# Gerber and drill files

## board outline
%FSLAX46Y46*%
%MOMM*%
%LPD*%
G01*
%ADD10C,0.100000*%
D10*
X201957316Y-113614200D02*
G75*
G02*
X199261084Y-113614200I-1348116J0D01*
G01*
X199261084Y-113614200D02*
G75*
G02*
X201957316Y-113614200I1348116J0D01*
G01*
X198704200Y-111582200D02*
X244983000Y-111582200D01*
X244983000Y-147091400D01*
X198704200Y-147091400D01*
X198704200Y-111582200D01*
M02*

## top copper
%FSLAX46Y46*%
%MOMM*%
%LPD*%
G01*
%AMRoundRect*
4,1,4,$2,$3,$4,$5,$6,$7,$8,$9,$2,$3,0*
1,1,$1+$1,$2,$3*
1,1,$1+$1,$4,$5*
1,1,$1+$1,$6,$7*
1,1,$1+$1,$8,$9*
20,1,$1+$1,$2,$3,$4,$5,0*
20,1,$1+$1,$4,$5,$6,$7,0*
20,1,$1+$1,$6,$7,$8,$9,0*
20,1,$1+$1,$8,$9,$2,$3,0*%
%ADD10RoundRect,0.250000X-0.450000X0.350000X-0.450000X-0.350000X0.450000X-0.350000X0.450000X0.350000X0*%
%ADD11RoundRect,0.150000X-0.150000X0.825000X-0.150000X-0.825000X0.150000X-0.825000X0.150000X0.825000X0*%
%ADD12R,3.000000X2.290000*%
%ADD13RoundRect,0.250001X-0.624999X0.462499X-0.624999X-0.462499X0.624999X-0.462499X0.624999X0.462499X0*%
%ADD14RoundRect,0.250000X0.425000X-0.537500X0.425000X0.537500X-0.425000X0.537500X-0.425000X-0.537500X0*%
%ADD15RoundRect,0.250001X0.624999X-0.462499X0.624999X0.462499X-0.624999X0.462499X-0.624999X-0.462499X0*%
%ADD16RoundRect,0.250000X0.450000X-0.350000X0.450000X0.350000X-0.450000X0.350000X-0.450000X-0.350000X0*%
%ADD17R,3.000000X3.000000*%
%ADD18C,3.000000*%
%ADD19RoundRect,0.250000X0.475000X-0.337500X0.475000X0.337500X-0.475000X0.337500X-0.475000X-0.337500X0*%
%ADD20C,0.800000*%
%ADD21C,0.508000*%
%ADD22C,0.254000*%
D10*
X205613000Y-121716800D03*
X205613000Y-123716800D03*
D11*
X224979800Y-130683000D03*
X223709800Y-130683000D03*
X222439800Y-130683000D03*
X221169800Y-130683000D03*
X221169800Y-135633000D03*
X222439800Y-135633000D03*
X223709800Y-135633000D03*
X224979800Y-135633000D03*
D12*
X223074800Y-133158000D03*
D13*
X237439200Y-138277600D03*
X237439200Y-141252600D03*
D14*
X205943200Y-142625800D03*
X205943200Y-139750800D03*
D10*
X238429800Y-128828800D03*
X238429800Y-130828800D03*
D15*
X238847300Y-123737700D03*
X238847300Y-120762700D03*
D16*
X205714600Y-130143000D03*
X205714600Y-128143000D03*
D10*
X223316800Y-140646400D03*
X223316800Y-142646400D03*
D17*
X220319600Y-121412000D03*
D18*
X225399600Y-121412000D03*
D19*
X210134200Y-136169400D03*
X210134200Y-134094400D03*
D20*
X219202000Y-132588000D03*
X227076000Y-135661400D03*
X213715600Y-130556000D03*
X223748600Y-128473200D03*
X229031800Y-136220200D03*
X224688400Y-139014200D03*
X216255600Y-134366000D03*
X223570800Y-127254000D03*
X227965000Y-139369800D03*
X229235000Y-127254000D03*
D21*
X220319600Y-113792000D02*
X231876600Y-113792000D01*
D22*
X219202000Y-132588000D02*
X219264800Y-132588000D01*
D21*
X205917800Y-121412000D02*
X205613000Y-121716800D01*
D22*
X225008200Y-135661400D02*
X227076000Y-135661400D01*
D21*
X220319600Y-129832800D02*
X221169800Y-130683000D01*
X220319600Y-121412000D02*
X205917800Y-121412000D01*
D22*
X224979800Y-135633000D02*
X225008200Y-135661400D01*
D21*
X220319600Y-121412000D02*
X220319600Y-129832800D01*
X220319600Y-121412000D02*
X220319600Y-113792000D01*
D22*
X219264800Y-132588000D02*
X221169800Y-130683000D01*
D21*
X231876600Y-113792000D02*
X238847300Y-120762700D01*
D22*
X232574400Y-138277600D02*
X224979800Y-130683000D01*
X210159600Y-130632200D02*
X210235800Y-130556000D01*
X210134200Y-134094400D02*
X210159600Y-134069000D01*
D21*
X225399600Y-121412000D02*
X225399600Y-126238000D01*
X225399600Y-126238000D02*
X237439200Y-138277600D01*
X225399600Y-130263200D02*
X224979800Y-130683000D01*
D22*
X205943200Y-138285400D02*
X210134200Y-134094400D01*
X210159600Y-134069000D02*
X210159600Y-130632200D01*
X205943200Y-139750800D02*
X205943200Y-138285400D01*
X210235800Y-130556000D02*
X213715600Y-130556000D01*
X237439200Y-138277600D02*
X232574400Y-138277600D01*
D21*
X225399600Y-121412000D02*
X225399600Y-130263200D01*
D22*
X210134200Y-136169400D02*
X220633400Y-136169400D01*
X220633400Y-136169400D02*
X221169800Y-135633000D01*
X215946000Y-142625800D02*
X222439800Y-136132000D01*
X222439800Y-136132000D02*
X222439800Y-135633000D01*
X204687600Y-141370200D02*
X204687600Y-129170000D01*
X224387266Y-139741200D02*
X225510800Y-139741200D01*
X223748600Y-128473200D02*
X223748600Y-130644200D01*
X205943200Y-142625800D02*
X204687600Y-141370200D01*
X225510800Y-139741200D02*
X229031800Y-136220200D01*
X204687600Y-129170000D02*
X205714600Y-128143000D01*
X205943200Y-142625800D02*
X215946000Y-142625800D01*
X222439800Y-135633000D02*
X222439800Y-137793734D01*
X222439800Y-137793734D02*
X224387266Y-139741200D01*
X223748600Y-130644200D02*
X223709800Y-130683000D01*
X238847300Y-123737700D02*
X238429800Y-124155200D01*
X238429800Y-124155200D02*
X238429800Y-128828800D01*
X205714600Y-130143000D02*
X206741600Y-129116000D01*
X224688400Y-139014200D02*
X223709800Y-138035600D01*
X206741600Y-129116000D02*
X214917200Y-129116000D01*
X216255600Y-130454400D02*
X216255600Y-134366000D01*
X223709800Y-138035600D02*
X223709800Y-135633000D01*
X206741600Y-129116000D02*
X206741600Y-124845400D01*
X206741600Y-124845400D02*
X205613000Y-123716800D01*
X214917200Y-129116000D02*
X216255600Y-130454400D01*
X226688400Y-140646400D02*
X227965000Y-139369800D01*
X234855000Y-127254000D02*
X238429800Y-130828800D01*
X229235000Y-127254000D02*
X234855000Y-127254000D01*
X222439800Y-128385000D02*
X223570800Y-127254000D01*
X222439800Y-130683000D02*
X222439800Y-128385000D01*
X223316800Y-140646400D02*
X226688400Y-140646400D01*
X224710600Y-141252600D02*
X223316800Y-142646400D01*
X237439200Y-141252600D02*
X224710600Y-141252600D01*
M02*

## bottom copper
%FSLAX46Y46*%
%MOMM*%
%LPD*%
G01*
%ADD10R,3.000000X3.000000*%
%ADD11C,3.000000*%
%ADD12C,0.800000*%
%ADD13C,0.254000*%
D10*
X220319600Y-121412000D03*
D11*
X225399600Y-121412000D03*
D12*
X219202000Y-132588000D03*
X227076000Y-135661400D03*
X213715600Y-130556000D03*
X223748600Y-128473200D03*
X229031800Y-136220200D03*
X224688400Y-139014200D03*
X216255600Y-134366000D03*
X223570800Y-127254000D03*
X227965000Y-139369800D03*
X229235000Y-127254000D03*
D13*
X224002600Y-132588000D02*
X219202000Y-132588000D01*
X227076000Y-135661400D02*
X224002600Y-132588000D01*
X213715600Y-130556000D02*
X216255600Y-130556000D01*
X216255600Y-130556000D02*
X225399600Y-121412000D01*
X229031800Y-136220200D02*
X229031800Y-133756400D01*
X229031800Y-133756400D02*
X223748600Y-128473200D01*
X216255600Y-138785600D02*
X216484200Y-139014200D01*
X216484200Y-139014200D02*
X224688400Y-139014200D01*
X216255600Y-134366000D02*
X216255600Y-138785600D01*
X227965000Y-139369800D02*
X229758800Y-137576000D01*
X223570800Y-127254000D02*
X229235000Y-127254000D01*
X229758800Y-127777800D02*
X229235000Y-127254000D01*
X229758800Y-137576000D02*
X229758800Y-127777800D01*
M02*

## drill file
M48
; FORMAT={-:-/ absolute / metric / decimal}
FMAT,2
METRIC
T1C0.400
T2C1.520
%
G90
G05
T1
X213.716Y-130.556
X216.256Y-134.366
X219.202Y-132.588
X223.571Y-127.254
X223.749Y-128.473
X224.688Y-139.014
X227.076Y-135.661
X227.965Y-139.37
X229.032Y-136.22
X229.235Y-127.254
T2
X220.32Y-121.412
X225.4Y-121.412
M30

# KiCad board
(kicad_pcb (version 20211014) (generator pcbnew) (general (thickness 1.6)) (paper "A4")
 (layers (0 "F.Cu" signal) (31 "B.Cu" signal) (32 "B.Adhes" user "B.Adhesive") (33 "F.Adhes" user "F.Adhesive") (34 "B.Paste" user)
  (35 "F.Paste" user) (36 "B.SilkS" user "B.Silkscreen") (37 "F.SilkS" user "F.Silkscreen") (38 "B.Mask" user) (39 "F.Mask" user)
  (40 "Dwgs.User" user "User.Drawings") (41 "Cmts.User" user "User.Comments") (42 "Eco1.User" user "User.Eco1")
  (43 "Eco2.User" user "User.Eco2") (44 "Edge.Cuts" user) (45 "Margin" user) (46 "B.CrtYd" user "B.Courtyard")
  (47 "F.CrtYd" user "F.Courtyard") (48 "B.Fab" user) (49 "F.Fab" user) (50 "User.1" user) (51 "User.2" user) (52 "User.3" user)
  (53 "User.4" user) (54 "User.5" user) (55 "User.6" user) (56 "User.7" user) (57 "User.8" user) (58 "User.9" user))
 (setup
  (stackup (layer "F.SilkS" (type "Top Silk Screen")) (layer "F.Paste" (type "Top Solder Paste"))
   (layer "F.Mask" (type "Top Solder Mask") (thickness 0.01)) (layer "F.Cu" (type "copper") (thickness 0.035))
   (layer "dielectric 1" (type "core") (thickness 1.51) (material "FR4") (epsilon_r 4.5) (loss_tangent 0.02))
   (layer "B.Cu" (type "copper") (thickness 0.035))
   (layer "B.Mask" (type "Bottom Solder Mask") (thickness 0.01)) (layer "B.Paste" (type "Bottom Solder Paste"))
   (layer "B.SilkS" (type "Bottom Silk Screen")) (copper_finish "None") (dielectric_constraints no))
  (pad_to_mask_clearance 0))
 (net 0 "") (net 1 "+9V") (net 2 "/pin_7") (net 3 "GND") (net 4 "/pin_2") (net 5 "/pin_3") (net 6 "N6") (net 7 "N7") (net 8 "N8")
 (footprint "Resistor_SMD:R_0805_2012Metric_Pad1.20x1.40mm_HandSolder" (layer "F.Cu") (at 205.613 122.7168 -90)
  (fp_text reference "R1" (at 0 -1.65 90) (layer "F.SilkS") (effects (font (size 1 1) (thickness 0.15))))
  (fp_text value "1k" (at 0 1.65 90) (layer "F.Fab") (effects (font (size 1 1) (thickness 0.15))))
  (pad "1" smd roundrect (at -1 0 270) (size 1.2 1.4) (layers "F.Cu" "F.Paste" "F.Mask") (roundrect_rratio 0.2083333333) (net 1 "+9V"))
  (pad "2" smd roundrect (at 1 0 270) (size 1.2 1.4) (layers "F.Cu" "F.Paste" "F.Mask") (roundrect_rratio 0.2083333333) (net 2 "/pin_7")))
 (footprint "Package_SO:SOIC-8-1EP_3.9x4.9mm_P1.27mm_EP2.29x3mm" (layer "F.Cu") (at 223.0748 133.158 -90)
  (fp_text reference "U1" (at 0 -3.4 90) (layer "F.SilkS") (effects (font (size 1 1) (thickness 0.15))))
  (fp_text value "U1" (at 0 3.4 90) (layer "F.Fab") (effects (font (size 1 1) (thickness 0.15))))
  (pad "" smd roundrect (at 0.57 -0.75 270) (size 0.92 1.21) (layers "F.Paste") (roundrect_rratio 0.25))
  (pad "" smd roundrect (at -0.57 0.75 270) (size 0.92 1.21) (layers "F.Paste") (roundrect_rratio 0.25))
  (pad "" smd roundrect (at 0.57 0.75 270) (size 0.92 1.21) (layers "F.Paste") (roundrect_rratio 0.25))
  (pad "" smd roundrect (at -0.57 -0.75 270) (size 0.92 1.21) (layers "F.Paste") (roundrect_rratio 0.25))
  (pad "1" smd roundrect (at -2.475 -1.905 270) (size 1.95 0.6) (layers "F.Cu" "F.Paste" "F.Mask") (roundrect_rratio 0.25) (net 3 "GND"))
  (pad "2" smd roundrect (at -2.475 -0.635 270) (size 1.95 0.6) (layers "F.Cu" "F.Paste" "F.Mask") (roundrect_rratio 0.25) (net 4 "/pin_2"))
  (pad "3" smd roundrect (at -2.475 0.635 270) (size 1.95 0.6) (layers "F.Cu" "F.Paste" "F.Mask") (roundrect_rratio 0.25) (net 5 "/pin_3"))
  (pad "4" smd roundrect (at -2.475 1.905 270) (size 1.95 0.6) (layers "F.Cu" "F.Paste" "F.Mask") (roundrect_rratio 0.25) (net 1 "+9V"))
  (pad "5" smd roundrect (at 2.475 1.905 270) (size 1.95 0.6) (layers "F.Cu" "F.Paste" "F.Mask") (roundrect_rratio 0.25) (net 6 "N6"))
  (pad "6" smd roundrect (at 2.475 0.635 270) (size 1.95 0.6) (layers "F.Cu" "F.Paste" "F.Mask") (roundrect_rratio 0.25) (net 4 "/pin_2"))
  (pad "7" smd roundrect (at 2.475 -0.635 270) (size 1.95 0.6) (layers "F.Cu" "F.Paste" "F.Mask") (roundrect_rratio 0.25) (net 2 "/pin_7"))
  (pad "8" smd roundrect (at 2.475 -1.905 270) (size 1.95 0.6) (layers "F.Cu" "F.Paste" "F.Mask") (roundrect_rratio 0.25) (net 1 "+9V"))
  (pad "9" smd rect (at 0 0 270) (size 2.29 3) (layers "F.Cu" "F.Mask")))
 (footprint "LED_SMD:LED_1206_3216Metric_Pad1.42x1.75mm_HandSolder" (layer "F.Cu") (at 237.4392 139.7651 -90)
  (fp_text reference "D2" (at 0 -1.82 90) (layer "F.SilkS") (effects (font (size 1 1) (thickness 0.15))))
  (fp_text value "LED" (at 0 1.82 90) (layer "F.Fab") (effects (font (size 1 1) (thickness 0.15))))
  (pad "1" smd roundrect (at -1.4875 0 270) (size 1.425 1.75) (layers "F.Cu" "F.Paste" "F.Mask") (roundrect_rratio 0.1754392982)
   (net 3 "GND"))
  (pad "2" smd roundrect (at 1.4875 0 270) (size 1.425 1.75) (layers "F.Cu" "F.Paste" "F.Mask") (roundrect_rratio 0.1754392982) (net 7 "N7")))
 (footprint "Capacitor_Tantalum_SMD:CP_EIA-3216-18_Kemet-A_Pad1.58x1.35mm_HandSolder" (layer "F.Cu") (at 205.9432 141.1883 90)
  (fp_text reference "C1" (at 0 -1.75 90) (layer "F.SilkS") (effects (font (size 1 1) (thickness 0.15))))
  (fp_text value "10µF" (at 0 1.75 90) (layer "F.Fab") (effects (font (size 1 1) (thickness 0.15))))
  (pad "1" smd roundrect (at -1.4375 0 90) (size 1.575 1.35) (layers "F.Cu" "F.Paste" "F.Mask") (roundrect_rratio 0.1851851852)
   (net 4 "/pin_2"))
  (pad "2" smd roundrect (at 1.4375 0 90) (size 1.575 1.35) (layers "F.Cu" "F.Paste" "F.Mask") (roundrect_rratio 0.1851851852) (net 3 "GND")))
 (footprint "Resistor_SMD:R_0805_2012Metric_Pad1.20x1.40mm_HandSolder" (layer "F.Cu") (at 238.4298 129.8288 -90)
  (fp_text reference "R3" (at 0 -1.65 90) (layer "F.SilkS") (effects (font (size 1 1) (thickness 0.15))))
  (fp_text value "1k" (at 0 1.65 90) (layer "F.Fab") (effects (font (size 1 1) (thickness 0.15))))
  (pad "1" smd roundrect (at -1 0 270) (size 1.2 1.4) (layers "F.Cu" "F.Paste" "F.Mask") (roundrect_rratio 0.2083333333) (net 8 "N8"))
  (pad "2" smd roundrect (at 1 0 270) (size 1.2 1.4) (layers "F.Cu" "F.Paste" "F.Mask") (roundrect_rratio 0.2083333333) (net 5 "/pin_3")))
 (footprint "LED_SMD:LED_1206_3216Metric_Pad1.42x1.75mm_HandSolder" (layer "F.Cu") (at 238.8473 122.2502 90)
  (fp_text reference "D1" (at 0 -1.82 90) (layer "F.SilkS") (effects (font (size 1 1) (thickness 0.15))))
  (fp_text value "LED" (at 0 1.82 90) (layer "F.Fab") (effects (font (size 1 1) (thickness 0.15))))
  (pad "1" smd roundrect (at -1.4875 0 90) (size 1.425 1.75) (layers "F.Cu" "F.Paste" "F.Mask") (roundrect_rratio 0.1754392982) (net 8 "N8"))
  (pad "2" smd roundrect (at 1.4875 0 90) (size 1.425 1.75) (layers "F.Cu" "F.Paste" "F.Mask") (roundrect_rratio 0.1754392982) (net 1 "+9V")))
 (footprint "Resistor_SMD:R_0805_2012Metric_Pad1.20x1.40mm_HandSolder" (layer "F.Cu") (at 205.7146 129.143 90)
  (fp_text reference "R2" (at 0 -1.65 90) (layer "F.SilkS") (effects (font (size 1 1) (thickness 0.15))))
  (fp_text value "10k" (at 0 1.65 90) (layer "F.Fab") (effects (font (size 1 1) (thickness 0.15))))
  (pad "1" smd roundrect (at -1 0 90) (size 1.2 1.4) (layers "F.Cu" "F.Paste" "F.Mask") (roundrect_rratio 0.2083333333) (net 2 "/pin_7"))
  (pad "2" smd roundrect (at 1 0 90) (size 1.2 1.4) (layers "F.Cu" "F.Paste" "F.Mask") (roundrect_rratio 0.2083333333) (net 4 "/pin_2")))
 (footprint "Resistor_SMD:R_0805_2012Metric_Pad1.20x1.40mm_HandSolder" (layer "F.Cu") (at 223.3168 141.6464 -90)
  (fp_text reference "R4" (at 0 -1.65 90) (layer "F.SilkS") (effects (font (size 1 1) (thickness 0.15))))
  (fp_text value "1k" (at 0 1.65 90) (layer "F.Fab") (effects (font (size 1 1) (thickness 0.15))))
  (pad "1" smd roundrect (at -1 0 270) (size 1.2 1.4) (layers "F.Cu" "F.Paste" "F.Mask") (roundrect_rratio 0.2083333333) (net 5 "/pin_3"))
  (pad "2" smd roundrect (at 1 0 270) (size 1.2 1.4) (layers "F.Cu" "F.Paste" "F.Mask") (roundrect_rratio 0.2083333333) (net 7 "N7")))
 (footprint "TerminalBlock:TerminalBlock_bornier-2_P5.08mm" (layer "F.Cu") (at 220.3196 121.412)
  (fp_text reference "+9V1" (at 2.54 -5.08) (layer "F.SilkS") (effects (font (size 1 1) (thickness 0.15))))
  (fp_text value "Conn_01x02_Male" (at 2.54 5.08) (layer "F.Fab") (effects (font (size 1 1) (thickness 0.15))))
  (pad "1" thru_hole rect (at 0 0) (size 3 3) (drill 1.52) (layers *.Cu *.Mask) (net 1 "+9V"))
  (pad "2" thru_hole circle (at 5.08 0) (size 3 3) (drill 1.52) (layers *.Cu *.Mask) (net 3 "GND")))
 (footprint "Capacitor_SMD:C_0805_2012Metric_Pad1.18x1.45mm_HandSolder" (layer "F.Cu") (at 210.1342 135.1319 90)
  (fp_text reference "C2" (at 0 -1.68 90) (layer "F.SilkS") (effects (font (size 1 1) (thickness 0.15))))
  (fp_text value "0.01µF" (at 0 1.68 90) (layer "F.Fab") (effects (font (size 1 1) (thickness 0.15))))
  (pad "1" smd roundrect (at -1.0375 0 90) (size 1.175 1.45) (layers "F.Cu" "F.Paste" "F.Mask") (roundrect_rratio 0.2127659574) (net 6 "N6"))
  (pad "2" smd roundrect (at 1.0375 0 90) (size 1.175 1.45) (layers "F.Cu" "F.Paste" "F.Mask") (roundrect_rratio 0.2127659574) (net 3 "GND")))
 (gr_circle (center 200.6092 113.6142) (end 201.957316 113.6142) (layer "Edge.Cuts") (width 0.1) (fill none))
 (gr_rect (start 198.7042 111.5822) (end 244.983 147.0914) (layer "Edge.Cuts") (width 0.1) (fill none))
 (segment (start 220.3196 113.792) (end 231.8766 113.792) (width 0.508) (layer "F.Cu") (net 1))
 (segment (start 219.202 132.588) (end 219.2648 132.588) (width 0.254) (layer "F.Cu") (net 1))
 (segment (start 205.9178 121.412) (end 205.613 121.7168) (width 0.508) (layer "F.Cu") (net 1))
 (segment (start 225.0082 135.6614) (end 227.076 135.6614) (width 0.254) (layer "F.Cu") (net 1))
 (segment (start 220.3196 129.8328) (end 221.1698 130.683) (width 0.508) (layer "F.Cu") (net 1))
 (segment (start 220.3196 121.412) (end 205.9178 121.412) (width 0.508) (layer "F.Cu") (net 1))
 (segment (start 224.9798 135.633) (end 225.0082 135.6614) (width 0.254) (layer "F.Cu") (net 1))
 (segment (start 220.3196 121.412) (end 220.3196 129.8328) (width 0.508) (layer "F.Cu") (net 1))
 (segment (start 220.3196 121.412) (end 220.3196 113.792) (width 0.508) (layer "F.Cu") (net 1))
 (segment (start 219.2648 132.588) (end 221.1698 130.683) (width 0.254) (layer "F.Cu") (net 1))
 (segment (start 231.8766 113.792) (end 238.8473 120.7627) (width 0.508) (layer "F.Cu") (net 1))
 (via (at 219.202 132.588) (size 0.8) (drill 0.4) (layers "F.Cu" "B.Cu") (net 1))
 (via (at 227.076 135.6614) (size 0.8) (drill 0.4) (layers "F.Cu" "B.Cu") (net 1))
 (segment (start 224.0026 132.588) (end 219.202 132.588) (width 0.254) (layer "B.Cu") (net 1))
 (segment (start 227.076 135.6614) (end 224.0026 132.588) (width 0.254) (layer "B.Cu") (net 1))
 (segment (start 232.5744 138.2776) (end 224.9798 130.683) (width 0.254) (layer "F.Cu") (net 3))
 (segment (start 210.1596 130.6322) (end 210.2358 130.556) (width 0.254) (layer "F.Cu") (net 3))
 (segment (start 210.1342 134.0944) (end 210.1596 134.069) (width 0.254) (layer "F.Cu") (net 3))
 (segment (start 225.3996 121.412) (end 225.3996 126.238) (width 0.508) (layer "F.Cu") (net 3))
 (segment (start 225.3996 126.238) (end 237.4392 138.2776) (width 0.508) (layer "F.Cu") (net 3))
 (segment (start 225.3996 130.2632) (end 224.9798 130.683) (width 0.508) (layer "F.Cu") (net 3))
 (segment (start 205.9432 138.2854) (end 210.1342 134.0944) (width 0.254) (layer "F.Cu") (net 3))
 (segment (start 210.1596 134.069) (end 210.1596 130.6322) (width 0.254) (layer "F.Cu") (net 3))
 (segment (start 205.9432 139.7508) (end 205.9432 138.2854) (width 0.254) (layer "F.Cu") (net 3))
 (segment (start 210.2358 130.556) (end 213.7156 130.556) (width 0.254) (layer "F.Cu") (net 3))
 (segment (start 237.4392 138.2776) (end 232.5744 138.2776) (width 0.254) (layer "F.Cu") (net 3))
 (segment (start 225.3996 121.412) (end 225.3996 130.2632) (width 0.508) (layer "F.Cu") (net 3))
 (via (at 213.7156 130.556) (size 0.8) (drill 0.4) (layers "F.Cu" "B.Cu") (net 3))
 (segment (start 213.7156 130.556) (end 216.2556 130.556) (width 0.254) (layer "B.Cu") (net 3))
 (segment (start 216.2556 130.556) (end 225.3996 121.412) (width 0.254) (layer "B.Cu") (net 3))
 (segment (start 210.1342 136.1694) (end 220.6334 136.1694) (width 0.254) (layer "F.Cu") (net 6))
 (segment (start 220.6334 136.1694) (end 221.1698 135.633) (width 0.254) (layer "F.Cu") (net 6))
 (segment (start 215.946 142.6258) (end 222.4398 136.132) (width 0.254) (layer "F.Cu") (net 4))
 (segment (start 222.4398 136.132) (end 222.4398 135.633) (width 0.254) (layer "F.Cu") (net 4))
 (segment (start 204.6876 141.3702) (end 204.6876 129.17) (width 0.254) (layer "F.Cu") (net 4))
 (segment (start 224.387266 139.7412) (end 225.5108 139.7412) (width 0.254) (layer "F.Cu") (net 4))
 (segment (start 223.7486 128.4732) (end 223.7486 130.6442) (width 0.254) (layer "F.Cu") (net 4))
 (segment (start 205.9432 142.6258) (end 204.6876 141.3702) (width 0.254) (layer "F.Cu") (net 4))
 (segment (start 225.5108 139.7412) (end 229.0318 136.2202) (width 0.254) (layer "F.Cu") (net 4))
 (segment (start 204.6876 129.17) (end 205.7146 128.143) (width 0.254) (layer "F.Cu") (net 4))
 (segment (start 205.9432 142.6258) (end 215.946 142.6258) (width 0.254) (layer "F.Cu") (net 4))
 (segment (start 222.4398 135.633) (end 222.4398 137.793734) (width 0.254) (layer "F.Cu") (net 4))
 (segment (start 222.4398 137.793734) (end 224.387266 139.7412) (width 0.254) (layer "F.Cu") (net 4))
 (segment (start 223.7486 130.6442) (end 223.7098 130.683) (width 0.254) (layer "F.Cu") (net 4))
 (via (at 223.7486 128.4732) (size 0.8) (drill 0.4) (layers "F.Cu" "B.Cu") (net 4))
 (via (at 229.0318 136.2202) (size 0.8) (drill 0.4) (layers "F.Cu" "B.Cu") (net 4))
 (segment (start 229.0318 136.2202) (end 229.0318 133.7564) (width 0.254) (layer "B.Cu") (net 4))
 (segment (start 229.0318 133.7564) (end 223.7486 128.4732) (width 0.254) (layer "B.Cu") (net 4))
 (segment (start 238.8473 123.7377) (end 238.4298 124.1552) (width 0.254) (layer "F.Cu") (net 8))
 (segment (start 238.4298 124.1552) (end 238.4298 128.8288) (width 0.254) (layer "F.Cu") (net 8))
 (segment (start 205.7146 130.143) (end 206.7416 129.116) (width 0.254) (layer "F.Cu") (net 2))
 (segment (start 224.6884 139.0142) (end 223.7098 138.0356) (width 0.254) (layer "F.Cu") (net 2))
 (segment (start 206.7416 129.116) (end 214.9172 129.116) (width 0.254) (layer "F.Cu") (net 2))
 (segment (start 216.2556 130.4544) (end 216.2556 134.366) (width 0.254) (layer "F.Cu") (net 2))
 (segment (start 223.7098 138.0356) (end 223.7098 135.633) (width 0.254) (layer "F.Cu") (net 2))
 (segment (start 206.7416 129.116) (end 206.7416 124.8454) (width 0.254) (layer "F.Cu") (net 2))
 (segment (start 206.7416 124.8454) (end 205.613 123.7168) (width 0.254) (layer "F.Cu") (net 2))
 (segment (start 214.9172 129.116) (end 216.2556 130.4544) (width 0.254) (layer "F.Cu") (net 2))
 (via (at 224.6884 139.0142) (size 0.8) (drill 0.4) (layers "F.Cu" "B.Cu") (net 2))
 (via (at 216.2556 134.366) (size 0.8) (drill 0.4) (layers "F.Cu" "B.Cu") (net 2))
 (segment (start 216.2556 138.7856) (end 216.4842 139.0142) (width 0.254) (layer "B.Cu") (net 2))
 (segment (start 216.4842 139.0142) (end 224.6884 139.0142) (width 0.254) (layer "B.Cu") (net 2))
 (segment (start 216.2556 134.366) (end 216.2556 138.7856) (width 0.254) (layer "B.Cu") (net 2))
 (segment (start 226.6884 140.6464) (end 227.965 139.3698) (width 0.254) (layer "F.Cu") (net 5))
 (segment (start 234.855 127.254) (end 238.4298 130.8288) (width 0.254) (layer "F.Cu") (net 5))
 (segment (start 229.235 127.254) (end 234.855 127.254) (width 0.254) (layer "F.Cu") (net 5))
 (segment (start 222.4398 128.385) (end 223.5708 127.254) (width 0.254) (layer "F.Cu") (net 5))
 (segment (start 222.4398 130.683) (end 222.4398 128.385) (width 0.254) (layer "F.Cu") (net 5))
 (segment (start 223.3168 140.6464) (end 226.6884 140.6464) (width 0.254) (layer "F.Cu") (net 5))
 (via (at 223.5708 127.254) (size 0.8) (drill 0.4) (layers "F.Cu" "B.Cu") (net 5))
 (via (at 227.965 139.3698) (size 0.8) (drill 0.4) (layers "F.Cu" "B.Cu") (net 5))
 (via (at 229.235 127.254) (size 0.8) (drill 0.4) (layers "F.Cu" "B.Cu") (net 5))
 (segment (start 227.965 139.3698) (end 229.7588 137.576) (width 0.254) (layer "B.Cu") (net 5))
 (segment (start 223.5708 127.254) (end 229.235 127.254) (width 0.254) (layer "B.Cu") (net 5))
 (segment (start 229.7588 127.7778) (end 229.235 127.254) (width 0.254) (layer "B.Cu") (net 5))
 (segment (start 229.7588 137.576) (end 229.7588 127.7778) (width 0.254) (layer "B.Cu") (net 5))
 (segment (start 224.7106 141.2526) (end 223.3168 142.6464) (width 0.254) (layer "F.Cu") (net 7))
 (segment (start 237.4392 141.2526) (end 224.7106 141.2526) (width 0.254) (layer "F.Cu") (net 7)))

